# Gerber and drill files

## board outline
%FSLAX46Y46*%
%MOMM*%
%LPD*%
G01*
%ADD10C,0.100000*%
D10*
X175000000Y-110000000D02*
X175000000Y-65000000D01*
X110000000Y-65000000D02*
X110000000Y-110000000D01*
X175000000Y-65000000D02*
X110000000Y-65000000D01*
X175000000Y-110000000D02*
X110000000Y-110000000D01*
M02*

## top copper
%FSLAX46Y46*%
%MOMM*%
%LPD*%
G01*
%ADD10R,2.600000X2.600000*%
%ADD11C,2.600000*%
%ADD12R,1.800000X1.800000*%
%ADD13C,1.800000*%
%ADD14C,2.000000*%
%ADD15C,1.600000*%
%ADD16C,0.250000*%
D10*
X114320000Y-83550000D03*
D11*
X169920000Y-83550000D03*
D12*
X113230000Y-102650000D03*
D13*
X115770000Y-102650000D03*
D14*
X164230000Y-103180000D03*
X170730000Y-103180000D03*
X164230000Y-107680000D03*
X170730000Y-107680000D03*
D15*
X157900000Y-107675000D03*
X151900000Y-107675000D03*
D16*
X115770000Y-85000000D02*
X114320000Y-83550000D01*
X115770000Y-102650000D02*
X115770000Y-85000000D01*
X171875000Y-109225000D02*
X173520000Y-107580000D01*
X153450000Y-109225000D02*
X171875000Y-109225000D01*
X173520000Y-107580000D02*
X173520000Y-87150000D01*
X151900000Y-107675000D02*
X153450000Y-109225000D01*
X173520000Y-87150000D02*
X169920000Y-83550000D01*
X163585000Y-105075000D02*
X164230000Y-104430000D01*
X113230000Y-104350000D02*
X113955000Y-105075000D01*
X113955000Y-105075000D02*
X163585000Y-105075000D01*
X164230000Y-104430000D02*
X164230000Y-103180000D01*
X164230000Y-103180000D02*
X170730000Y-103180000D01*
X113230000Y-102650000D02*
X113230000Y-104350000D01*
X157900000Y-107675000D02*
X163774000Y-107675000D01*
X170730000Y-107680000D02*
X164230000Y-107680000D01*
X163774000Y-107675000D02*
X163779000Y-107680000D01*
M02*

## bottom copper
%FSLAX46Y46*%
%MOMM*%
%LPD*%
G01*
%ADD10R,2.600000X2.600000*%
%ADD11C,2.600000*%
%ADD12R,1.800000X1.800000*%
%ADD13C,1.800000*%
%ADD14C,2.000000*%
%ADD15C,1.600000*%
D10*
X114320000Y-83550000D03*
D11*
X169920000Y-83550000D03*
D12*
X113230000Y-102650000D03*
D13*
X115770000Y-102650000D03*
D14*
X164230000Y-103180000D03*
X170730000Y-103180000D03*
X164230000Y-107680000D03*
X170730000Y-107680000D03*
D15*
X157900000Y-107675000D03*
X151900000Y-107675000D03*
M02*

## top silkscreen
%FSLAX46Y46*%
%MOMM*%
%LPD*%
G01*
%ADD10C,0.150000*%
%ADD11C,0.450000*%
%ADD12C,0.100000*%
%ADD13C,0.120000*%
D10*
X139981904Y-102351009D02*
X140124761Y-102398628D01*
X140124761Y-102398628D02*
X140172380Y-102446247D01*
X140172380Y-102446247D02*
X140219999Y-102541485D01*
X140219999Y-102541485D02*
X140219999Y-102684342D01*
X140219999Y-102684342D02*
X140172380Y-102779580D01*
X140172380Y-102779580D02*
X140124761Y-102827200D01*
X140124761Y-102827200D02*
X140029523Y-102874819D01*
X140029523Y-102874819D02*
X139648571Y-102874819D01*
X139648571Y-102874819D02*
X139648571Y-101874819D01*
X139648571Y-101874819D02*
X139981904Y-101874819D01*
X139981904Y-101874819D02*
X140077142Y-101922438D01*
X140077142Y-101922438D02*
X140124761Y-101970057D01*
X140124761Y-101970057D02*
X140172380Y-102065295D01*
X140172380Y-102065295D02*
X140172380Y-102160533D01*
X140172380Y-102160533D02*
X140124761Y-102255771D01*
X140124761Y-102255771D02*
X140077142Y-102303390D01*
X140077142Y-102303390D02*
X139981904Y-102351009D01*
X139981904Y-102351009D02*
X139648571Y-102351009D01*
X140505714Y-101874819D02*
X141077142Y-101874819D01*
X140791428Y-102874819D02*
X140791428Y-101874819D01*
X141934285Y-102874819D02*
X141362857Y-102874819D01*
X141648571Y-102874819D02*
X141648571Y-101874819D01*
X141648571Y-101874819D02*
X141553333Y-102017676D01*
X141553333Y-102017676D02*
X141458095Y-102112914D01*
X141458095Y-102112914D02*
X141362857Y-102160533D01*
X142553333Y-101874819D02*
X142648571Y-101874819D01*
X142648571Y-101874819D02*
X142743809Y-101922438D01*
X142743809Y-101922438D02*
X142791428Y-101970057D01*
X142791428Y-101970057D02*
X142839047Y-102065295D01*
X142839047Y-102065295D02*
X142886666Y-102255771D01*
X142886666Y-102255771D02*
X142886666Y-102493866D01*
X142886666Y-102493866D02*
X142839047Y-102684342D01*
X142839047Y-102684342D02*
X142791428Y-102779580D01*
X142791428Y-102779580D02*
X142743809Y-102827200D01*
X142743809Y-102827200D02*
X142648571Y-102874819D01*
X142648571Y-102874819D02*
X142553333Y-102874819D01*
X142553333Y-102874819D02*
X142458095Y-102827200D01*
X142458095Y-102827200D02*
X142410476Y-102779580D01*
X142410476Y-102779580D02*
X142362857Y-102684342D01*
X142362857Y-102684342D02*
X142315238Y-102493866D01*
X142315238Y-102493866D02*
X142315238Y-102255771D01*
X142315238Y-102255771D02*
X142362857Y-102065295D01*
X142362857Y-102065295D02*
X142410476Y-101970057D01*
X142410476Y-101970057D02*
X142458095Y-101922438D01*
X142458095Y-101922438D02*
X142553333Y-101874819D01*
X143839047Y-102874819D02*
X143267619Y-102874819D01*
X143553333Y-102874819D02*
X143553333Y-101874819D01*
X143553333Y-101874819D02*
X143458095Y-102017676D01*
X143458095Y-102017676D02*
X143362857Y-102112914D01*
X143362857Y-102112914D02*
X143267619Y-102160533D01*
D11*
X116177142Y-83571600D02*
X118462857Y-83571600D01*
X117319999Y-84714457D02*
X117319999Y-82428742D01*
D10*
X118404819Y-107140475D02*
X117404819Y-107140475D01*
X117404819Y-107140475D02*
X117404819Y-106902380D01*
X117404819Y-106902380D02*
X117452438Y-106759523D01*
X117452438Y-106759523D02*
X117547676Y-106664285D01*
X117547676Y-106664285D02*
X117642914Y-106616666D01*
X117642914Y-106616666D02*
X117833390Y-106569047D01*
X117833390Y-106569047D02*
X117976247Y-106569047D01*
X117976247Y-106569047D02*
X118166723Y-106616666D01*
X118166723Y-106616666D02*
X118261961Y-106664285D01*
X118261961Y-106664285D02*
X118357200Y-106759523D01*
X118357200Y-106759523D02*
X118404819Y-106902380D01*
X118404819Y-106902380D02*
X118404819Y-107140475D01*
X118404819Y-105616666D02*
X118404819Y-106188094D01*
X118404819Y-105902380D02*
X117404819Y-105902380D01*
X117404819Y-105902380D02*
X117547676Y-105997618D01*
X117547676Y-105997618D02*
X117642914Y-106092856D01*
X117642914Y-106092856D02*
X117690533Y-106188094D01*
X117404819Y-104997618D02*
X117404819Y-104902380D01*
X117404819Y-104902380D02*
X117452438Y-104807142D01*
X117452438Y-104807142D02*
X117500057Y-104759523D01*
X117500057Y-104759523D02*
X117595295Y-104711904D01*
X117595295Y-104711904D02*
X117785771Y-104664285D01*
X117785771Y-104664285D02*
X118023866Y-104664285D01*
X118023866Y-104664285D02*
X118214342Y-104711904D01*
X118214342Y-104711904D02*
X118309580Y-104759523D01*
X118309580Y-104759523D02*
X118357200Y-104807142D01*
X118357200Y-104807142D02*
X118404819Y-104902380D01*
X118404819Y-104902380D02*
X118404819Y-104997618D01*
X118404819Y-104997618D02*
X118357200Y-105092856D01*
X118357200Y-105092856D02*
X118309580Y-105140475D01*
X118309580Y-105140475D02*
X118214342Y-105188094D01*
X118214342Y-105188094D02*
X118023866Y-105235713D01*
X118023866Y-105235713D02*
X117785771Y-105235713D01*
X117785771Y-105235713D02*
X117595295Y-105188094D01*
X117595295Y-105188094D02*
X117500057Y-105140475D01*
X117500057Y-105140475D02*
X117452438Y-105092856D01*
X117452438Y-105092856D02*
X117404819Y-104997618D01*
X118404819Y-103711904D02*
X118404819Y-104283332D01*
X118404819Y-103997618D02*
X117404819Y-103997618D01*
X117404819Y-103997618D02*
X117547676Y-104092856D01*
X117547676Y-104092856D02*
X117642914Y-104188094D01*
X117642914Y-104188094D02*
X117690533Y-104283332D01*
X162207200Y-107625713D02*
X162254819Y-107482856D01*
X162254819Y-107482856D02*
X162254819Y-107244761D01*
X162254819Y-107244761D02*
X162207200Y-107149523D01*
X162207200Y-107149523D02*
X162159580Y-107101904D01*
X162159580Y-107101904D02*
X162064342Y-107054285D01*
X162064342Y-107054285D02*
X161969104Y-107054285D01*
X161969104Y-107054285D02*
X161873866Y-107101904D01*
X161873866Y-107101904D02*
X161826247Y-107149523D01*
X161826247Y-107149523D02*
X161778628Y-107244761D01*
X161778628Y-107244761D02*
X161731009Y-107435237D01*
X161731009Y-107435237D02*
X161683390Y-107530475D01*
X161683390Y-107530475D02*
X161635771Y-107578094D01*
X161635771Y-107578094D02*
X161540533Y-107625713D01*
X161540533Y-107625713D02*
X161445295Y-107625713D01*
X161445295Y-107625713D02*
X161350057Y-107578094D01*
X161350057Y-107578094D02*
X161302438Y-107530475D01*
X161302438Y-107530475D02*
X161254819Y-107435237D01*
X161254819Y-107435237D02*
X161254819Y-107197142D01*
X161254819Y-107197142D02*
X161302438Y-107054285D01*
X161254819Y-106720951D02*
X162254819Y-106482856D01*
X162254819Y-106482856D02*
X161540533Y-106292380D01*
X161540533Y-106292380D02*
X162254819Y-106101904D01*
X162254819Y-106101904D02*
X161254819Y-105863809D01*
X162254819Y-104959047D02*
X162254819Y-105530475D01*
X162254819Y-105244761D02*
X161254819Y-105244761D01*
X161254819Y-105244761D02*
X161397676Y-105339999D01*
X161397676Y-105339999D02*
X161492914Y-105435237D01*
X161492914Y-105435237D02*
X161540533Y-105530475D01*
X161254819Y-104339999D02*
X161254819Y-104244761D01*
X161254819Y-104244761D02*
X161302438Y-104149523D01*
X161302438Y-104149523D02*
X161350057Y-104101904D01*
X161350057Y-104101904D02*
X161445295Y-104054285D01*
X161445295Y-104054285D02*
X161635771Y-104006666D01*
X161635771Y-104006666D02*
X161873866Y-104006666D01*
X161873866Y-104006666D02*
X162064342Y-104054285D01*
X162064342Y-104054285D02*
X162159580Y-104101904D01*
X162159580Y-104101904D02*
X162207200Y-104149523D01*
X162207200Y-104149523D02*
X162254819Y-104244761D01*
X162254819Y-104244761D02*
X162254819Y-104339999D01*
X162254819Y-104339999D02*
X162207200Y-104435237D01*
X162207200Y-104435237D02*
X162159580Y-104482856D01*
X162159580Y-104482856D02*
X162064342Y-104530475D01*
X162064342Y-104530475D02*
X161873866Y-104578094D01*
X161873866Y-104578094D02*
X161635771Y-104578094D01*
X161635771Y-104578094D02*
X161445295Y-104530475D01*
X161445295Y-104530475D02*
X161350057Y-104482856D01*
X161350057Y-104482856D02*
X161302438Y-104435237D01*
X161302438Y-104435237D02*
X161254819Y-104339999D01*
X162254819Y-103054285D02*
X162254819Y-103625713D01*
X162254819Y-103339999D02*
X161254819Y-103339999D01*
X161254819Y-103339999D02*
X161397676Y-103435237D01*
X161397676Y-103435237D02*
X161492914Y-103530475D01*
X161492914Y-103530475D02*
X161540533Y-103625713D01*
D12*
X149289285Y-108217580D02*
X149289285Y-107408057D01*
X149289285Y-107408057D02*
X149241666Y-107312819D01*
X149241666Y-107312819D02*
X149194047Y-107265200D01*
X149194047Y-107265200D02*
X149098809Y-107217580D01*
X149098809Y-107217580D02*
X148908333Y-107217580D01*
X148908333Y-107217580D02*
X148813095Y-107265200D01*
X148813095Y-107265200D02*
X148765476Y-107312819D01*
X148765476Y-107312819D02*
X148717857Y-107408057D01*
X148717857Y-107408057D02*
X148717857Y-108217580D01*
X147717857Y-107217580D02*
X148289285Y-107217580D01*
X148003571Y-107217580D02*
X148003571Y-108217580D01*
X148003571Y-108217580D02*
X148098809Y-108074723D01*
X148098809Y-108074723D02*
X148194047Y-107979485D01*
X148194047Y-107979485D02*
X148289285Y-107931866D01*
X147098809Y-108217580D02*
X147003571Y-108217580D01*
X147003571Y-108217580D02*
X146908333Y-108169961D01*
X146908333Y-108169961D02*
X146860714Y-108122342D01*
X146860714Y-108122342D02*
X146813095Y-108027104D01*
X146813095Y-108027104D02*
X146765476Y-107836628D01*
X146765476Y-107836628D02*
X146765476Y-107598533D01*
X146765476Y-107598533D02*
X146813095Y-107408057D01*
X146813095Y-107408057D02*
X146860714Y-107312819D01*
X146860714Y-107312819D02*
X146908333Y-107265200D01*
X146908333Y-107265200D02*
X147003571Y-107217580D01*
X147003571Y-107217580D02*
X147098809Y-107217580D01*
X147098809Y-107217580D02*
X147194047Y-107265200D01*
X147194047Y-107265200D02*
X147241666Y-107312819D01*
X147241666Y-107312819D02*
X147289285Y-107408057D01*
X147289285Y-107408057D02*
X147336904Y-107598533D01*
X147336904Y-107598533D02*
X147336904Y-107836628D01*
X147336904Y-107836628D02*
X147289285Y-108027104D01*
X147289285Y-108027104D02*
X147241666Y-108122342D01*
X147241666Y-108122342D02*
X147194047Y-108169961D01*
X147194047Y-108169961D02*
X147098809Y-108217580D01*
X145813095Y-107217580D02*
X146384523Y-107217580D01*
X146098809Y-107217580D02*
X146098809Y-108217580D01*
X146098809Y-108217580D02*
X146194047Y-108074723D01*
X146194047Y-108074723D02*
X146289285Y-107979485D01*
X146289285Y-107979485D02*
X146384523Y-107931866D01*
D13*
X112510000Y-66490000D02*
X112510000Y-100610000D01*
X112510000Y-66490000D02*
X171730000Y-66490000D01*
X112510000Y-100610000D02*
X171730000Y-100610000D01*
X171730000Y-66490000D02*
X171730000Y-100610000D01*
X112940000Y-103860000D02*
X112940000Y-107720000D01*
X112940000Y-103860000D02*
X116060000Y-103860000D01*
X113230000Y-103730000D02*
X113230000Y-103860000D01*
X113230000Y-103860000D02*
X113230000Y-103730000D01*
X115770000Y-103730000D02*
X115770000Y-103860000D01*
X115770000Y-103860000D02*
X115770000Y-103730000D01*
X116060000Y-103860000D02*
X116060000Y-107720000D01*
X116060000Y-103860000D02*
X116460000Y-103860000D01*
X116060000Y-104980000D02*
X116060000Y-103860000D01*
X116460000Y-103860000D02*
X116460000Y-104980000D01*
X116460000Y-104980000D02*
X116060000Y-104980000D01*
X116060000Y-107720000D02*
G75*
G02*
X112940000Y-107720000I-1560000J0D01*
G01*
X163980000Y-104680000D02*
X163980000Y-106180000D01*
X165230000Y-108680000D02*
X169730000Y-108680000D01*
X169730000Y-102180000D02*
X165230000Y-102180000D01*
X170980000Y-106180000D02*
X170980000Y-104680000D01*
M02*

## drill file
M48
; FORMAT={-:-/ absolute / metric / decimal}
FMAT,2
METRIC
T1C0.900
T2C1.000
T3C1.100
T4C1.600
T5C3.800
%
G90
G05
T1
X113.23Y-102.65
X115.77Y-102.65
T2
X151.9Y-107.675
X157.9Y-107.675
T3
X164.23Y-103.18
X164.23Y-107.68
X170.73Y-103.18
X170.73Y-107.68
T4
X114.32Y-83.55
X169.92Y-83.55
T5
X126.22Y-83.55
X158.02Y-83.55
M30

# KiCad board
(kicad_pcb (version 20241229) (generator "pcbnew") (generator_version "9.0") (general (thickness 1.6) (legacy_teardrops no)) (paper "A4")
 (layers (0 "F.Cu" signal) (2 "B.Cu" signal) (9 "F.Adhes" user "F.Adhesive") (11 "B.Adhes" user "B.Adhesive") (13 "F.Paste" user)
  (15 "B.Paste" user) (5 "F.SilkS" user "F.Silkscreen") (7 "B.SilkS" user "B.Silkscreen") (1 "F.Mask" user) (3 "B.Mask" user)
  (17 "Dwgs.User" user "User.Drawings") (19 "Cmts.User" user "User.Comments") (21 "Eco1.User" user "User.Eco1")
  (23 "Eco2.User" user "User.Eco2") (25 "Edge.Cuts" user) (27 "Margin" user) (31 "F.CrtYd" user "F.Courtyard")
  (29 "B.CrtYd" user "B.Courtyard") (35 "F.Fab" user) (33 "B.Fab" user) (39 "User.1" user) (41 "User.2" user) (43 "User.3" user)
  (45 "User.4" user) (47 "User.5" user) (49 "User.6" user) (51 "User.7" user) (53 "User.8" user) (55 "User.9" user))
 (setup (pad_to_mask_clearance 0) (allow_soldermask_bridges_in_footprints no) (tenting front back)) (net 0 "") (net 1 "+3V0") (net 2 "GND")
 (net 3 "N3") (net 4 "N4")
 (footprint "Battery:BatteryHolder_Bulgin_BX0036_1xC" (layer "F.Cu") (at 114.32 83.55)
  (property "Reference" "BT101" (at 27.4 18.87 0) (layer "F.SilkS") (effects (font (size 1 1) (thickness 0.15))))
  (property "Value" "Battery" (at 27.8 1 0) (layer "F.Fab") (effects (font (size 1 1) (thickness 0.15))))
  (fp_line (start -1.81 -17.06) (end -1.81 17.06) (stroke (width 0.12) (type solid)) (layer "F.SilkS"))
  (fp_line (start -1.81 -17.06) (end 57.41 -17.06) (stroke (width 0.12) (type solid)) (layer "F.SilkS"))
  (fp_line (start -1.81 17.06) (end 57.41 17.06) (stroke (width 0.12) (type solid)) (layer "F.SilkS"))
  (fp_line (start 57.41 -17.06) (end 57.41 17.06) (stroke (width 0.12) (type solid)) (layer "F.SilkS"))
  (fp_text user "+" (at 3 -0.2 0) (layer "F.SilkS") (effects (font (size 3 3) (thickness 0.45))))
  (pad "" np_thru_hole circle (at 11.9 0) (size 3.8 3.8) (drill 3.8) (layers "*.Cu" "*.Mask"))
  (pad "" np_thru_hole circle (at 43.7 0) (size 3.8 3.8) (drill 3.8) (layers "*.Cu" "*.Mask"))
  (pad "1" thru_hole rect (at 0 0) (size 2.6 2.6) (drill 1.6) (layers "*.Cu" "*.Mask") (remove_unused_layers no) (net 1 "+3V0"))
  (pad "2" thru_hole circle (at 55.6 0) (size 2.6 2.6) (drill 1.6) (layers "*.Cu" "*.Mask") (remove_unused_layers no) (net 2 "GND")))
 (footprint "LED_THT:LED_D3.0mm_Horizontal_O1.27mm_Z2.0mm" (layer "F.Cu") (at 113.23 102.65)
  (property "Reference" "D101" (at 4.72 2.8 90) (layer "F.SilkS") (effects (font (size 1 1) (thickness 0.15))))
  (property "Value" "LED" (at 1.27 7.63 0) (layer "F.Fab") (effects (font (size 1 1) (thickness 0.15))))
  (fp_line (start -0.29 1.21) (end -0.29 5.07) (stroke (width 0.12) (type solid)) (layer "F.SilkS"))
  (fp_line (start -0.29 1.21) (end 2.83 1.21) (stroke (width 0.12) (type solid)) (layer "F.SilkS"))
  (fp_line (start 0 1.08) (end 0 1.21) (stroke (width 0.12) (type solid)) (layer "F.SilkS"))
  (fp_line (start 0 1.21) (end 0 1.08) (stroke (width 0.12) (type solid)) (layer "F.SilkS"))
  (fp_line (start 2.54 1.08) (end 2.54 1.21) (stroke (width 0.12) (type solid)) (layer "F.SilkS"))
  (fp_line (start 2.54 1.21) (end 2.54 1.08) (stroke (width 0.12) (type solid)) (layer "F.SilkS"))
  (fp_line (start 2.83 1.21) (end 2.83 5.07) (stroke (width 0.12) (type solid)) (layer "F.SilkS"))
  (fp_line (start 2.83 1.21) (end 3.23 1.21) (stroke (width 0.12) (type solid)) (layer "F.SilkS"))
  (fp_line (start 2.83 2.33) (end 2.83 1.21) (stroke (width 0.12) (type solid)) (layer "F.SilkS"))
  (fp_line (start 3.23 1.21) (end 3.23 2.33) (stroke (width 0.12) (type solid)) (layer "F.SilkS"))
  (fp_line (start 3.23 2.33) (end 2.83 2.33) (stroke (width 0.12) (type solid)) (layer "F.SilkS"))
  (fp_arc (start 2.83 5.07) (mid 1.27 6.63) (end -0.29 5.07) (stroke (width 0.12) (type solid)) (layer "F.SilkS"))
  (pad "1" thru_hole rect (at 0 0) (size 1.8 1.8) (drill 0.9) (layers "*.Cu" "*.Mask") (remove_unused_layers no) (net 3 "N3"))
  (pad "2" thru_hole circle (at 2.54 0) (size 1.8 1.8) (drill 0.9) (layers "*.Cu" "*.Mask") (remove_unused_layers no) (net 1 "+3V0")))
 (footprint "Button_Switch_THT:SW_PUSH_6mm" (layer "F.Cu") (at 164.23 103.18)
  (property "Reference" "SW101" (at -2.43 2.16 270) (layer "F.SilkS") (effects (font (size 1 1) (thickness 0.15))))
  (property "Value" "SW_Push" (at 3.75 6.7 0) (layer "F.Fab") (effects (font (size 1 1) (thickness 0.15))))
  (fp_line (start -0.25 1.5) (end -0.25 3) (stroke (width 0.12) (type solid)) (layer "F.SilkS"))
  (fp_line (start 1 5.5) (end 5.5 5.5) (stroke (width 0.12) (type solid)) (layer "F.SilkS"))
  (fp_line (start 5.5 -1) (end 1 -1) (stroke (width 0.12) (type solid)) (layer "F.SilkS"))
  (fp_line (start 6.75 3) (end 6.75 1.5) (stroke (width 0.12) (type solid)) (layer "F.SilkS"))
  (pad "1" thru_hole circle (at 0 0 90) (size 2 2) (drill 1.1) (layers "*.Cu" "*.Mask") (remove_unused_layers no) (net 3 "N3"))
  (pad "1" thru_hole circle (at 6.5 0 90) (size 2 2) (drill 1.1) (layers "*.Cu" "*.Mask") (remove_unused_layers no) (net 3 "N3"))
  (pad "2" thru_hole circle (at 0 4.5 90) (size 2 2) (drill 1.1) (layers "*.Cu" "*.Mask") (remove_unused_layers no) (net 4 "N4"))
  (pad "2" thru_hole circle (at 6.5 4.5 90) (size 2 2) (drill 1.1) (layers "*.Cu" "*.Mask") (remove_unused_layers no) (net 4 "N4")))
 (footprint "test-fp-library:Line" (layer "F.Cu") (at 154.9 107.675 180)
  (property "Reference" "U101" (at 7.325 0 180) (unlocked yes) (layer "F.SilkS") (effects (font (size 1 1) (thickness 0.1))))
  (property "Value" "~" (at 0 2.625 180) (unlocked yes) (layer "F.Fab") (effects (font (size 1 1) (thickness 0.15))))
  (pad "1" thru_hole circle (at -3 0 180) (size 1.6 1.6) (drill 1) (layers "*.Cu" "*.Mask") (remove_unused_layers no) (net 4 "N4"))
  (pad "2" thru_hole circle (at 3 0 180) (size 1.6 1.6) (drill 1) (layers "*.Cu" "*.Mask") (remove_unused_layers no) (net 2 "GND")))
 (gr_line (start 175 110) (end 175 65) (stroke (width 0.1) (type default)) (layer "Edge.Cuts"))
 (gr_line (start 110 65) (end 110 110) (stroke (width 0.1) (type default)) (layer "Edge.Cuts"))
 (gr_line (start 175 65) (end 110 65) (stroke (width 0.1) (type default)) (layer "Edge.Cuts"))
 (gr_line (start 175 110) (end 110 110) (stroke (width 0.1) (type default)) (layer "Edge.Cuts"))
 (segment (start 115.77 85) (end 114.32 83.55) (width 0.25) (layer "F.Cu") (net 1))
 (segment (start 115.77 102.65) (end 115.77 85) (width 0.25) (layer "F.Cu") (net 1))
 (segment (start 171.875 109.225) (end 173.52 107.58) (width 0.25) (layer "F.Cu") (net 2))
 (segment (start 153.45 109.225) (end 171.875 109.225) (width 0.25) (layer "F.Cu") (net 2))
 (segment (start 173.52 107.58) (end 173.52 87.15) (width 0.25) (layer "F.Cu") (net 2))
 (segment (start 151.9 107.675) (end 153.45 109.225) (width 0.25) (layer "F.Cu") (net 2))
 (segment (start 173.52 87.15) (end 169.92 83.55) (width 0.25) (layer "F.Cu") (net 2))
 (segment (start 163.585 105.075) (end 164.23 104.43) (width 0.25) (layer "F.Cu") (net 3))
 (segment (start 113.23 104.35) (end 113.955 105.075) (width 0.25) (layer "F.Cu") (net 3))
 (segment (start 113.955 105.075) (end 163.585 105.075) (width 0.25) (layer "F.Cu") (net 3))
 (segment (start 164.23 104.43) (end 164.23 103.18) (width 0.25) (layer "F.Cu") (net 3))
 (segment (start 164.23 103.18) (end 170.73 103.18) (width 0.25) (layer "F.Cu") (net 3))
 (segment (start 113.23 102.65) (end 113.23 104.35) (width 0.25) (layer "F.Cu") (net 3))
 (segment (start 157.9 107.675) (end 163.774 107.675) (width 0.25) (layer "F.Cu") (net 4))
 (segment (start 170.73 107.68) (end 164.23 107.68) (width 0.25) (layer "F.Cu") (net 4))
 (segment (start 163.774 107.675) (end 163.779 107.68) (width 0.25) (layer "F.Cu") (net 4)))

